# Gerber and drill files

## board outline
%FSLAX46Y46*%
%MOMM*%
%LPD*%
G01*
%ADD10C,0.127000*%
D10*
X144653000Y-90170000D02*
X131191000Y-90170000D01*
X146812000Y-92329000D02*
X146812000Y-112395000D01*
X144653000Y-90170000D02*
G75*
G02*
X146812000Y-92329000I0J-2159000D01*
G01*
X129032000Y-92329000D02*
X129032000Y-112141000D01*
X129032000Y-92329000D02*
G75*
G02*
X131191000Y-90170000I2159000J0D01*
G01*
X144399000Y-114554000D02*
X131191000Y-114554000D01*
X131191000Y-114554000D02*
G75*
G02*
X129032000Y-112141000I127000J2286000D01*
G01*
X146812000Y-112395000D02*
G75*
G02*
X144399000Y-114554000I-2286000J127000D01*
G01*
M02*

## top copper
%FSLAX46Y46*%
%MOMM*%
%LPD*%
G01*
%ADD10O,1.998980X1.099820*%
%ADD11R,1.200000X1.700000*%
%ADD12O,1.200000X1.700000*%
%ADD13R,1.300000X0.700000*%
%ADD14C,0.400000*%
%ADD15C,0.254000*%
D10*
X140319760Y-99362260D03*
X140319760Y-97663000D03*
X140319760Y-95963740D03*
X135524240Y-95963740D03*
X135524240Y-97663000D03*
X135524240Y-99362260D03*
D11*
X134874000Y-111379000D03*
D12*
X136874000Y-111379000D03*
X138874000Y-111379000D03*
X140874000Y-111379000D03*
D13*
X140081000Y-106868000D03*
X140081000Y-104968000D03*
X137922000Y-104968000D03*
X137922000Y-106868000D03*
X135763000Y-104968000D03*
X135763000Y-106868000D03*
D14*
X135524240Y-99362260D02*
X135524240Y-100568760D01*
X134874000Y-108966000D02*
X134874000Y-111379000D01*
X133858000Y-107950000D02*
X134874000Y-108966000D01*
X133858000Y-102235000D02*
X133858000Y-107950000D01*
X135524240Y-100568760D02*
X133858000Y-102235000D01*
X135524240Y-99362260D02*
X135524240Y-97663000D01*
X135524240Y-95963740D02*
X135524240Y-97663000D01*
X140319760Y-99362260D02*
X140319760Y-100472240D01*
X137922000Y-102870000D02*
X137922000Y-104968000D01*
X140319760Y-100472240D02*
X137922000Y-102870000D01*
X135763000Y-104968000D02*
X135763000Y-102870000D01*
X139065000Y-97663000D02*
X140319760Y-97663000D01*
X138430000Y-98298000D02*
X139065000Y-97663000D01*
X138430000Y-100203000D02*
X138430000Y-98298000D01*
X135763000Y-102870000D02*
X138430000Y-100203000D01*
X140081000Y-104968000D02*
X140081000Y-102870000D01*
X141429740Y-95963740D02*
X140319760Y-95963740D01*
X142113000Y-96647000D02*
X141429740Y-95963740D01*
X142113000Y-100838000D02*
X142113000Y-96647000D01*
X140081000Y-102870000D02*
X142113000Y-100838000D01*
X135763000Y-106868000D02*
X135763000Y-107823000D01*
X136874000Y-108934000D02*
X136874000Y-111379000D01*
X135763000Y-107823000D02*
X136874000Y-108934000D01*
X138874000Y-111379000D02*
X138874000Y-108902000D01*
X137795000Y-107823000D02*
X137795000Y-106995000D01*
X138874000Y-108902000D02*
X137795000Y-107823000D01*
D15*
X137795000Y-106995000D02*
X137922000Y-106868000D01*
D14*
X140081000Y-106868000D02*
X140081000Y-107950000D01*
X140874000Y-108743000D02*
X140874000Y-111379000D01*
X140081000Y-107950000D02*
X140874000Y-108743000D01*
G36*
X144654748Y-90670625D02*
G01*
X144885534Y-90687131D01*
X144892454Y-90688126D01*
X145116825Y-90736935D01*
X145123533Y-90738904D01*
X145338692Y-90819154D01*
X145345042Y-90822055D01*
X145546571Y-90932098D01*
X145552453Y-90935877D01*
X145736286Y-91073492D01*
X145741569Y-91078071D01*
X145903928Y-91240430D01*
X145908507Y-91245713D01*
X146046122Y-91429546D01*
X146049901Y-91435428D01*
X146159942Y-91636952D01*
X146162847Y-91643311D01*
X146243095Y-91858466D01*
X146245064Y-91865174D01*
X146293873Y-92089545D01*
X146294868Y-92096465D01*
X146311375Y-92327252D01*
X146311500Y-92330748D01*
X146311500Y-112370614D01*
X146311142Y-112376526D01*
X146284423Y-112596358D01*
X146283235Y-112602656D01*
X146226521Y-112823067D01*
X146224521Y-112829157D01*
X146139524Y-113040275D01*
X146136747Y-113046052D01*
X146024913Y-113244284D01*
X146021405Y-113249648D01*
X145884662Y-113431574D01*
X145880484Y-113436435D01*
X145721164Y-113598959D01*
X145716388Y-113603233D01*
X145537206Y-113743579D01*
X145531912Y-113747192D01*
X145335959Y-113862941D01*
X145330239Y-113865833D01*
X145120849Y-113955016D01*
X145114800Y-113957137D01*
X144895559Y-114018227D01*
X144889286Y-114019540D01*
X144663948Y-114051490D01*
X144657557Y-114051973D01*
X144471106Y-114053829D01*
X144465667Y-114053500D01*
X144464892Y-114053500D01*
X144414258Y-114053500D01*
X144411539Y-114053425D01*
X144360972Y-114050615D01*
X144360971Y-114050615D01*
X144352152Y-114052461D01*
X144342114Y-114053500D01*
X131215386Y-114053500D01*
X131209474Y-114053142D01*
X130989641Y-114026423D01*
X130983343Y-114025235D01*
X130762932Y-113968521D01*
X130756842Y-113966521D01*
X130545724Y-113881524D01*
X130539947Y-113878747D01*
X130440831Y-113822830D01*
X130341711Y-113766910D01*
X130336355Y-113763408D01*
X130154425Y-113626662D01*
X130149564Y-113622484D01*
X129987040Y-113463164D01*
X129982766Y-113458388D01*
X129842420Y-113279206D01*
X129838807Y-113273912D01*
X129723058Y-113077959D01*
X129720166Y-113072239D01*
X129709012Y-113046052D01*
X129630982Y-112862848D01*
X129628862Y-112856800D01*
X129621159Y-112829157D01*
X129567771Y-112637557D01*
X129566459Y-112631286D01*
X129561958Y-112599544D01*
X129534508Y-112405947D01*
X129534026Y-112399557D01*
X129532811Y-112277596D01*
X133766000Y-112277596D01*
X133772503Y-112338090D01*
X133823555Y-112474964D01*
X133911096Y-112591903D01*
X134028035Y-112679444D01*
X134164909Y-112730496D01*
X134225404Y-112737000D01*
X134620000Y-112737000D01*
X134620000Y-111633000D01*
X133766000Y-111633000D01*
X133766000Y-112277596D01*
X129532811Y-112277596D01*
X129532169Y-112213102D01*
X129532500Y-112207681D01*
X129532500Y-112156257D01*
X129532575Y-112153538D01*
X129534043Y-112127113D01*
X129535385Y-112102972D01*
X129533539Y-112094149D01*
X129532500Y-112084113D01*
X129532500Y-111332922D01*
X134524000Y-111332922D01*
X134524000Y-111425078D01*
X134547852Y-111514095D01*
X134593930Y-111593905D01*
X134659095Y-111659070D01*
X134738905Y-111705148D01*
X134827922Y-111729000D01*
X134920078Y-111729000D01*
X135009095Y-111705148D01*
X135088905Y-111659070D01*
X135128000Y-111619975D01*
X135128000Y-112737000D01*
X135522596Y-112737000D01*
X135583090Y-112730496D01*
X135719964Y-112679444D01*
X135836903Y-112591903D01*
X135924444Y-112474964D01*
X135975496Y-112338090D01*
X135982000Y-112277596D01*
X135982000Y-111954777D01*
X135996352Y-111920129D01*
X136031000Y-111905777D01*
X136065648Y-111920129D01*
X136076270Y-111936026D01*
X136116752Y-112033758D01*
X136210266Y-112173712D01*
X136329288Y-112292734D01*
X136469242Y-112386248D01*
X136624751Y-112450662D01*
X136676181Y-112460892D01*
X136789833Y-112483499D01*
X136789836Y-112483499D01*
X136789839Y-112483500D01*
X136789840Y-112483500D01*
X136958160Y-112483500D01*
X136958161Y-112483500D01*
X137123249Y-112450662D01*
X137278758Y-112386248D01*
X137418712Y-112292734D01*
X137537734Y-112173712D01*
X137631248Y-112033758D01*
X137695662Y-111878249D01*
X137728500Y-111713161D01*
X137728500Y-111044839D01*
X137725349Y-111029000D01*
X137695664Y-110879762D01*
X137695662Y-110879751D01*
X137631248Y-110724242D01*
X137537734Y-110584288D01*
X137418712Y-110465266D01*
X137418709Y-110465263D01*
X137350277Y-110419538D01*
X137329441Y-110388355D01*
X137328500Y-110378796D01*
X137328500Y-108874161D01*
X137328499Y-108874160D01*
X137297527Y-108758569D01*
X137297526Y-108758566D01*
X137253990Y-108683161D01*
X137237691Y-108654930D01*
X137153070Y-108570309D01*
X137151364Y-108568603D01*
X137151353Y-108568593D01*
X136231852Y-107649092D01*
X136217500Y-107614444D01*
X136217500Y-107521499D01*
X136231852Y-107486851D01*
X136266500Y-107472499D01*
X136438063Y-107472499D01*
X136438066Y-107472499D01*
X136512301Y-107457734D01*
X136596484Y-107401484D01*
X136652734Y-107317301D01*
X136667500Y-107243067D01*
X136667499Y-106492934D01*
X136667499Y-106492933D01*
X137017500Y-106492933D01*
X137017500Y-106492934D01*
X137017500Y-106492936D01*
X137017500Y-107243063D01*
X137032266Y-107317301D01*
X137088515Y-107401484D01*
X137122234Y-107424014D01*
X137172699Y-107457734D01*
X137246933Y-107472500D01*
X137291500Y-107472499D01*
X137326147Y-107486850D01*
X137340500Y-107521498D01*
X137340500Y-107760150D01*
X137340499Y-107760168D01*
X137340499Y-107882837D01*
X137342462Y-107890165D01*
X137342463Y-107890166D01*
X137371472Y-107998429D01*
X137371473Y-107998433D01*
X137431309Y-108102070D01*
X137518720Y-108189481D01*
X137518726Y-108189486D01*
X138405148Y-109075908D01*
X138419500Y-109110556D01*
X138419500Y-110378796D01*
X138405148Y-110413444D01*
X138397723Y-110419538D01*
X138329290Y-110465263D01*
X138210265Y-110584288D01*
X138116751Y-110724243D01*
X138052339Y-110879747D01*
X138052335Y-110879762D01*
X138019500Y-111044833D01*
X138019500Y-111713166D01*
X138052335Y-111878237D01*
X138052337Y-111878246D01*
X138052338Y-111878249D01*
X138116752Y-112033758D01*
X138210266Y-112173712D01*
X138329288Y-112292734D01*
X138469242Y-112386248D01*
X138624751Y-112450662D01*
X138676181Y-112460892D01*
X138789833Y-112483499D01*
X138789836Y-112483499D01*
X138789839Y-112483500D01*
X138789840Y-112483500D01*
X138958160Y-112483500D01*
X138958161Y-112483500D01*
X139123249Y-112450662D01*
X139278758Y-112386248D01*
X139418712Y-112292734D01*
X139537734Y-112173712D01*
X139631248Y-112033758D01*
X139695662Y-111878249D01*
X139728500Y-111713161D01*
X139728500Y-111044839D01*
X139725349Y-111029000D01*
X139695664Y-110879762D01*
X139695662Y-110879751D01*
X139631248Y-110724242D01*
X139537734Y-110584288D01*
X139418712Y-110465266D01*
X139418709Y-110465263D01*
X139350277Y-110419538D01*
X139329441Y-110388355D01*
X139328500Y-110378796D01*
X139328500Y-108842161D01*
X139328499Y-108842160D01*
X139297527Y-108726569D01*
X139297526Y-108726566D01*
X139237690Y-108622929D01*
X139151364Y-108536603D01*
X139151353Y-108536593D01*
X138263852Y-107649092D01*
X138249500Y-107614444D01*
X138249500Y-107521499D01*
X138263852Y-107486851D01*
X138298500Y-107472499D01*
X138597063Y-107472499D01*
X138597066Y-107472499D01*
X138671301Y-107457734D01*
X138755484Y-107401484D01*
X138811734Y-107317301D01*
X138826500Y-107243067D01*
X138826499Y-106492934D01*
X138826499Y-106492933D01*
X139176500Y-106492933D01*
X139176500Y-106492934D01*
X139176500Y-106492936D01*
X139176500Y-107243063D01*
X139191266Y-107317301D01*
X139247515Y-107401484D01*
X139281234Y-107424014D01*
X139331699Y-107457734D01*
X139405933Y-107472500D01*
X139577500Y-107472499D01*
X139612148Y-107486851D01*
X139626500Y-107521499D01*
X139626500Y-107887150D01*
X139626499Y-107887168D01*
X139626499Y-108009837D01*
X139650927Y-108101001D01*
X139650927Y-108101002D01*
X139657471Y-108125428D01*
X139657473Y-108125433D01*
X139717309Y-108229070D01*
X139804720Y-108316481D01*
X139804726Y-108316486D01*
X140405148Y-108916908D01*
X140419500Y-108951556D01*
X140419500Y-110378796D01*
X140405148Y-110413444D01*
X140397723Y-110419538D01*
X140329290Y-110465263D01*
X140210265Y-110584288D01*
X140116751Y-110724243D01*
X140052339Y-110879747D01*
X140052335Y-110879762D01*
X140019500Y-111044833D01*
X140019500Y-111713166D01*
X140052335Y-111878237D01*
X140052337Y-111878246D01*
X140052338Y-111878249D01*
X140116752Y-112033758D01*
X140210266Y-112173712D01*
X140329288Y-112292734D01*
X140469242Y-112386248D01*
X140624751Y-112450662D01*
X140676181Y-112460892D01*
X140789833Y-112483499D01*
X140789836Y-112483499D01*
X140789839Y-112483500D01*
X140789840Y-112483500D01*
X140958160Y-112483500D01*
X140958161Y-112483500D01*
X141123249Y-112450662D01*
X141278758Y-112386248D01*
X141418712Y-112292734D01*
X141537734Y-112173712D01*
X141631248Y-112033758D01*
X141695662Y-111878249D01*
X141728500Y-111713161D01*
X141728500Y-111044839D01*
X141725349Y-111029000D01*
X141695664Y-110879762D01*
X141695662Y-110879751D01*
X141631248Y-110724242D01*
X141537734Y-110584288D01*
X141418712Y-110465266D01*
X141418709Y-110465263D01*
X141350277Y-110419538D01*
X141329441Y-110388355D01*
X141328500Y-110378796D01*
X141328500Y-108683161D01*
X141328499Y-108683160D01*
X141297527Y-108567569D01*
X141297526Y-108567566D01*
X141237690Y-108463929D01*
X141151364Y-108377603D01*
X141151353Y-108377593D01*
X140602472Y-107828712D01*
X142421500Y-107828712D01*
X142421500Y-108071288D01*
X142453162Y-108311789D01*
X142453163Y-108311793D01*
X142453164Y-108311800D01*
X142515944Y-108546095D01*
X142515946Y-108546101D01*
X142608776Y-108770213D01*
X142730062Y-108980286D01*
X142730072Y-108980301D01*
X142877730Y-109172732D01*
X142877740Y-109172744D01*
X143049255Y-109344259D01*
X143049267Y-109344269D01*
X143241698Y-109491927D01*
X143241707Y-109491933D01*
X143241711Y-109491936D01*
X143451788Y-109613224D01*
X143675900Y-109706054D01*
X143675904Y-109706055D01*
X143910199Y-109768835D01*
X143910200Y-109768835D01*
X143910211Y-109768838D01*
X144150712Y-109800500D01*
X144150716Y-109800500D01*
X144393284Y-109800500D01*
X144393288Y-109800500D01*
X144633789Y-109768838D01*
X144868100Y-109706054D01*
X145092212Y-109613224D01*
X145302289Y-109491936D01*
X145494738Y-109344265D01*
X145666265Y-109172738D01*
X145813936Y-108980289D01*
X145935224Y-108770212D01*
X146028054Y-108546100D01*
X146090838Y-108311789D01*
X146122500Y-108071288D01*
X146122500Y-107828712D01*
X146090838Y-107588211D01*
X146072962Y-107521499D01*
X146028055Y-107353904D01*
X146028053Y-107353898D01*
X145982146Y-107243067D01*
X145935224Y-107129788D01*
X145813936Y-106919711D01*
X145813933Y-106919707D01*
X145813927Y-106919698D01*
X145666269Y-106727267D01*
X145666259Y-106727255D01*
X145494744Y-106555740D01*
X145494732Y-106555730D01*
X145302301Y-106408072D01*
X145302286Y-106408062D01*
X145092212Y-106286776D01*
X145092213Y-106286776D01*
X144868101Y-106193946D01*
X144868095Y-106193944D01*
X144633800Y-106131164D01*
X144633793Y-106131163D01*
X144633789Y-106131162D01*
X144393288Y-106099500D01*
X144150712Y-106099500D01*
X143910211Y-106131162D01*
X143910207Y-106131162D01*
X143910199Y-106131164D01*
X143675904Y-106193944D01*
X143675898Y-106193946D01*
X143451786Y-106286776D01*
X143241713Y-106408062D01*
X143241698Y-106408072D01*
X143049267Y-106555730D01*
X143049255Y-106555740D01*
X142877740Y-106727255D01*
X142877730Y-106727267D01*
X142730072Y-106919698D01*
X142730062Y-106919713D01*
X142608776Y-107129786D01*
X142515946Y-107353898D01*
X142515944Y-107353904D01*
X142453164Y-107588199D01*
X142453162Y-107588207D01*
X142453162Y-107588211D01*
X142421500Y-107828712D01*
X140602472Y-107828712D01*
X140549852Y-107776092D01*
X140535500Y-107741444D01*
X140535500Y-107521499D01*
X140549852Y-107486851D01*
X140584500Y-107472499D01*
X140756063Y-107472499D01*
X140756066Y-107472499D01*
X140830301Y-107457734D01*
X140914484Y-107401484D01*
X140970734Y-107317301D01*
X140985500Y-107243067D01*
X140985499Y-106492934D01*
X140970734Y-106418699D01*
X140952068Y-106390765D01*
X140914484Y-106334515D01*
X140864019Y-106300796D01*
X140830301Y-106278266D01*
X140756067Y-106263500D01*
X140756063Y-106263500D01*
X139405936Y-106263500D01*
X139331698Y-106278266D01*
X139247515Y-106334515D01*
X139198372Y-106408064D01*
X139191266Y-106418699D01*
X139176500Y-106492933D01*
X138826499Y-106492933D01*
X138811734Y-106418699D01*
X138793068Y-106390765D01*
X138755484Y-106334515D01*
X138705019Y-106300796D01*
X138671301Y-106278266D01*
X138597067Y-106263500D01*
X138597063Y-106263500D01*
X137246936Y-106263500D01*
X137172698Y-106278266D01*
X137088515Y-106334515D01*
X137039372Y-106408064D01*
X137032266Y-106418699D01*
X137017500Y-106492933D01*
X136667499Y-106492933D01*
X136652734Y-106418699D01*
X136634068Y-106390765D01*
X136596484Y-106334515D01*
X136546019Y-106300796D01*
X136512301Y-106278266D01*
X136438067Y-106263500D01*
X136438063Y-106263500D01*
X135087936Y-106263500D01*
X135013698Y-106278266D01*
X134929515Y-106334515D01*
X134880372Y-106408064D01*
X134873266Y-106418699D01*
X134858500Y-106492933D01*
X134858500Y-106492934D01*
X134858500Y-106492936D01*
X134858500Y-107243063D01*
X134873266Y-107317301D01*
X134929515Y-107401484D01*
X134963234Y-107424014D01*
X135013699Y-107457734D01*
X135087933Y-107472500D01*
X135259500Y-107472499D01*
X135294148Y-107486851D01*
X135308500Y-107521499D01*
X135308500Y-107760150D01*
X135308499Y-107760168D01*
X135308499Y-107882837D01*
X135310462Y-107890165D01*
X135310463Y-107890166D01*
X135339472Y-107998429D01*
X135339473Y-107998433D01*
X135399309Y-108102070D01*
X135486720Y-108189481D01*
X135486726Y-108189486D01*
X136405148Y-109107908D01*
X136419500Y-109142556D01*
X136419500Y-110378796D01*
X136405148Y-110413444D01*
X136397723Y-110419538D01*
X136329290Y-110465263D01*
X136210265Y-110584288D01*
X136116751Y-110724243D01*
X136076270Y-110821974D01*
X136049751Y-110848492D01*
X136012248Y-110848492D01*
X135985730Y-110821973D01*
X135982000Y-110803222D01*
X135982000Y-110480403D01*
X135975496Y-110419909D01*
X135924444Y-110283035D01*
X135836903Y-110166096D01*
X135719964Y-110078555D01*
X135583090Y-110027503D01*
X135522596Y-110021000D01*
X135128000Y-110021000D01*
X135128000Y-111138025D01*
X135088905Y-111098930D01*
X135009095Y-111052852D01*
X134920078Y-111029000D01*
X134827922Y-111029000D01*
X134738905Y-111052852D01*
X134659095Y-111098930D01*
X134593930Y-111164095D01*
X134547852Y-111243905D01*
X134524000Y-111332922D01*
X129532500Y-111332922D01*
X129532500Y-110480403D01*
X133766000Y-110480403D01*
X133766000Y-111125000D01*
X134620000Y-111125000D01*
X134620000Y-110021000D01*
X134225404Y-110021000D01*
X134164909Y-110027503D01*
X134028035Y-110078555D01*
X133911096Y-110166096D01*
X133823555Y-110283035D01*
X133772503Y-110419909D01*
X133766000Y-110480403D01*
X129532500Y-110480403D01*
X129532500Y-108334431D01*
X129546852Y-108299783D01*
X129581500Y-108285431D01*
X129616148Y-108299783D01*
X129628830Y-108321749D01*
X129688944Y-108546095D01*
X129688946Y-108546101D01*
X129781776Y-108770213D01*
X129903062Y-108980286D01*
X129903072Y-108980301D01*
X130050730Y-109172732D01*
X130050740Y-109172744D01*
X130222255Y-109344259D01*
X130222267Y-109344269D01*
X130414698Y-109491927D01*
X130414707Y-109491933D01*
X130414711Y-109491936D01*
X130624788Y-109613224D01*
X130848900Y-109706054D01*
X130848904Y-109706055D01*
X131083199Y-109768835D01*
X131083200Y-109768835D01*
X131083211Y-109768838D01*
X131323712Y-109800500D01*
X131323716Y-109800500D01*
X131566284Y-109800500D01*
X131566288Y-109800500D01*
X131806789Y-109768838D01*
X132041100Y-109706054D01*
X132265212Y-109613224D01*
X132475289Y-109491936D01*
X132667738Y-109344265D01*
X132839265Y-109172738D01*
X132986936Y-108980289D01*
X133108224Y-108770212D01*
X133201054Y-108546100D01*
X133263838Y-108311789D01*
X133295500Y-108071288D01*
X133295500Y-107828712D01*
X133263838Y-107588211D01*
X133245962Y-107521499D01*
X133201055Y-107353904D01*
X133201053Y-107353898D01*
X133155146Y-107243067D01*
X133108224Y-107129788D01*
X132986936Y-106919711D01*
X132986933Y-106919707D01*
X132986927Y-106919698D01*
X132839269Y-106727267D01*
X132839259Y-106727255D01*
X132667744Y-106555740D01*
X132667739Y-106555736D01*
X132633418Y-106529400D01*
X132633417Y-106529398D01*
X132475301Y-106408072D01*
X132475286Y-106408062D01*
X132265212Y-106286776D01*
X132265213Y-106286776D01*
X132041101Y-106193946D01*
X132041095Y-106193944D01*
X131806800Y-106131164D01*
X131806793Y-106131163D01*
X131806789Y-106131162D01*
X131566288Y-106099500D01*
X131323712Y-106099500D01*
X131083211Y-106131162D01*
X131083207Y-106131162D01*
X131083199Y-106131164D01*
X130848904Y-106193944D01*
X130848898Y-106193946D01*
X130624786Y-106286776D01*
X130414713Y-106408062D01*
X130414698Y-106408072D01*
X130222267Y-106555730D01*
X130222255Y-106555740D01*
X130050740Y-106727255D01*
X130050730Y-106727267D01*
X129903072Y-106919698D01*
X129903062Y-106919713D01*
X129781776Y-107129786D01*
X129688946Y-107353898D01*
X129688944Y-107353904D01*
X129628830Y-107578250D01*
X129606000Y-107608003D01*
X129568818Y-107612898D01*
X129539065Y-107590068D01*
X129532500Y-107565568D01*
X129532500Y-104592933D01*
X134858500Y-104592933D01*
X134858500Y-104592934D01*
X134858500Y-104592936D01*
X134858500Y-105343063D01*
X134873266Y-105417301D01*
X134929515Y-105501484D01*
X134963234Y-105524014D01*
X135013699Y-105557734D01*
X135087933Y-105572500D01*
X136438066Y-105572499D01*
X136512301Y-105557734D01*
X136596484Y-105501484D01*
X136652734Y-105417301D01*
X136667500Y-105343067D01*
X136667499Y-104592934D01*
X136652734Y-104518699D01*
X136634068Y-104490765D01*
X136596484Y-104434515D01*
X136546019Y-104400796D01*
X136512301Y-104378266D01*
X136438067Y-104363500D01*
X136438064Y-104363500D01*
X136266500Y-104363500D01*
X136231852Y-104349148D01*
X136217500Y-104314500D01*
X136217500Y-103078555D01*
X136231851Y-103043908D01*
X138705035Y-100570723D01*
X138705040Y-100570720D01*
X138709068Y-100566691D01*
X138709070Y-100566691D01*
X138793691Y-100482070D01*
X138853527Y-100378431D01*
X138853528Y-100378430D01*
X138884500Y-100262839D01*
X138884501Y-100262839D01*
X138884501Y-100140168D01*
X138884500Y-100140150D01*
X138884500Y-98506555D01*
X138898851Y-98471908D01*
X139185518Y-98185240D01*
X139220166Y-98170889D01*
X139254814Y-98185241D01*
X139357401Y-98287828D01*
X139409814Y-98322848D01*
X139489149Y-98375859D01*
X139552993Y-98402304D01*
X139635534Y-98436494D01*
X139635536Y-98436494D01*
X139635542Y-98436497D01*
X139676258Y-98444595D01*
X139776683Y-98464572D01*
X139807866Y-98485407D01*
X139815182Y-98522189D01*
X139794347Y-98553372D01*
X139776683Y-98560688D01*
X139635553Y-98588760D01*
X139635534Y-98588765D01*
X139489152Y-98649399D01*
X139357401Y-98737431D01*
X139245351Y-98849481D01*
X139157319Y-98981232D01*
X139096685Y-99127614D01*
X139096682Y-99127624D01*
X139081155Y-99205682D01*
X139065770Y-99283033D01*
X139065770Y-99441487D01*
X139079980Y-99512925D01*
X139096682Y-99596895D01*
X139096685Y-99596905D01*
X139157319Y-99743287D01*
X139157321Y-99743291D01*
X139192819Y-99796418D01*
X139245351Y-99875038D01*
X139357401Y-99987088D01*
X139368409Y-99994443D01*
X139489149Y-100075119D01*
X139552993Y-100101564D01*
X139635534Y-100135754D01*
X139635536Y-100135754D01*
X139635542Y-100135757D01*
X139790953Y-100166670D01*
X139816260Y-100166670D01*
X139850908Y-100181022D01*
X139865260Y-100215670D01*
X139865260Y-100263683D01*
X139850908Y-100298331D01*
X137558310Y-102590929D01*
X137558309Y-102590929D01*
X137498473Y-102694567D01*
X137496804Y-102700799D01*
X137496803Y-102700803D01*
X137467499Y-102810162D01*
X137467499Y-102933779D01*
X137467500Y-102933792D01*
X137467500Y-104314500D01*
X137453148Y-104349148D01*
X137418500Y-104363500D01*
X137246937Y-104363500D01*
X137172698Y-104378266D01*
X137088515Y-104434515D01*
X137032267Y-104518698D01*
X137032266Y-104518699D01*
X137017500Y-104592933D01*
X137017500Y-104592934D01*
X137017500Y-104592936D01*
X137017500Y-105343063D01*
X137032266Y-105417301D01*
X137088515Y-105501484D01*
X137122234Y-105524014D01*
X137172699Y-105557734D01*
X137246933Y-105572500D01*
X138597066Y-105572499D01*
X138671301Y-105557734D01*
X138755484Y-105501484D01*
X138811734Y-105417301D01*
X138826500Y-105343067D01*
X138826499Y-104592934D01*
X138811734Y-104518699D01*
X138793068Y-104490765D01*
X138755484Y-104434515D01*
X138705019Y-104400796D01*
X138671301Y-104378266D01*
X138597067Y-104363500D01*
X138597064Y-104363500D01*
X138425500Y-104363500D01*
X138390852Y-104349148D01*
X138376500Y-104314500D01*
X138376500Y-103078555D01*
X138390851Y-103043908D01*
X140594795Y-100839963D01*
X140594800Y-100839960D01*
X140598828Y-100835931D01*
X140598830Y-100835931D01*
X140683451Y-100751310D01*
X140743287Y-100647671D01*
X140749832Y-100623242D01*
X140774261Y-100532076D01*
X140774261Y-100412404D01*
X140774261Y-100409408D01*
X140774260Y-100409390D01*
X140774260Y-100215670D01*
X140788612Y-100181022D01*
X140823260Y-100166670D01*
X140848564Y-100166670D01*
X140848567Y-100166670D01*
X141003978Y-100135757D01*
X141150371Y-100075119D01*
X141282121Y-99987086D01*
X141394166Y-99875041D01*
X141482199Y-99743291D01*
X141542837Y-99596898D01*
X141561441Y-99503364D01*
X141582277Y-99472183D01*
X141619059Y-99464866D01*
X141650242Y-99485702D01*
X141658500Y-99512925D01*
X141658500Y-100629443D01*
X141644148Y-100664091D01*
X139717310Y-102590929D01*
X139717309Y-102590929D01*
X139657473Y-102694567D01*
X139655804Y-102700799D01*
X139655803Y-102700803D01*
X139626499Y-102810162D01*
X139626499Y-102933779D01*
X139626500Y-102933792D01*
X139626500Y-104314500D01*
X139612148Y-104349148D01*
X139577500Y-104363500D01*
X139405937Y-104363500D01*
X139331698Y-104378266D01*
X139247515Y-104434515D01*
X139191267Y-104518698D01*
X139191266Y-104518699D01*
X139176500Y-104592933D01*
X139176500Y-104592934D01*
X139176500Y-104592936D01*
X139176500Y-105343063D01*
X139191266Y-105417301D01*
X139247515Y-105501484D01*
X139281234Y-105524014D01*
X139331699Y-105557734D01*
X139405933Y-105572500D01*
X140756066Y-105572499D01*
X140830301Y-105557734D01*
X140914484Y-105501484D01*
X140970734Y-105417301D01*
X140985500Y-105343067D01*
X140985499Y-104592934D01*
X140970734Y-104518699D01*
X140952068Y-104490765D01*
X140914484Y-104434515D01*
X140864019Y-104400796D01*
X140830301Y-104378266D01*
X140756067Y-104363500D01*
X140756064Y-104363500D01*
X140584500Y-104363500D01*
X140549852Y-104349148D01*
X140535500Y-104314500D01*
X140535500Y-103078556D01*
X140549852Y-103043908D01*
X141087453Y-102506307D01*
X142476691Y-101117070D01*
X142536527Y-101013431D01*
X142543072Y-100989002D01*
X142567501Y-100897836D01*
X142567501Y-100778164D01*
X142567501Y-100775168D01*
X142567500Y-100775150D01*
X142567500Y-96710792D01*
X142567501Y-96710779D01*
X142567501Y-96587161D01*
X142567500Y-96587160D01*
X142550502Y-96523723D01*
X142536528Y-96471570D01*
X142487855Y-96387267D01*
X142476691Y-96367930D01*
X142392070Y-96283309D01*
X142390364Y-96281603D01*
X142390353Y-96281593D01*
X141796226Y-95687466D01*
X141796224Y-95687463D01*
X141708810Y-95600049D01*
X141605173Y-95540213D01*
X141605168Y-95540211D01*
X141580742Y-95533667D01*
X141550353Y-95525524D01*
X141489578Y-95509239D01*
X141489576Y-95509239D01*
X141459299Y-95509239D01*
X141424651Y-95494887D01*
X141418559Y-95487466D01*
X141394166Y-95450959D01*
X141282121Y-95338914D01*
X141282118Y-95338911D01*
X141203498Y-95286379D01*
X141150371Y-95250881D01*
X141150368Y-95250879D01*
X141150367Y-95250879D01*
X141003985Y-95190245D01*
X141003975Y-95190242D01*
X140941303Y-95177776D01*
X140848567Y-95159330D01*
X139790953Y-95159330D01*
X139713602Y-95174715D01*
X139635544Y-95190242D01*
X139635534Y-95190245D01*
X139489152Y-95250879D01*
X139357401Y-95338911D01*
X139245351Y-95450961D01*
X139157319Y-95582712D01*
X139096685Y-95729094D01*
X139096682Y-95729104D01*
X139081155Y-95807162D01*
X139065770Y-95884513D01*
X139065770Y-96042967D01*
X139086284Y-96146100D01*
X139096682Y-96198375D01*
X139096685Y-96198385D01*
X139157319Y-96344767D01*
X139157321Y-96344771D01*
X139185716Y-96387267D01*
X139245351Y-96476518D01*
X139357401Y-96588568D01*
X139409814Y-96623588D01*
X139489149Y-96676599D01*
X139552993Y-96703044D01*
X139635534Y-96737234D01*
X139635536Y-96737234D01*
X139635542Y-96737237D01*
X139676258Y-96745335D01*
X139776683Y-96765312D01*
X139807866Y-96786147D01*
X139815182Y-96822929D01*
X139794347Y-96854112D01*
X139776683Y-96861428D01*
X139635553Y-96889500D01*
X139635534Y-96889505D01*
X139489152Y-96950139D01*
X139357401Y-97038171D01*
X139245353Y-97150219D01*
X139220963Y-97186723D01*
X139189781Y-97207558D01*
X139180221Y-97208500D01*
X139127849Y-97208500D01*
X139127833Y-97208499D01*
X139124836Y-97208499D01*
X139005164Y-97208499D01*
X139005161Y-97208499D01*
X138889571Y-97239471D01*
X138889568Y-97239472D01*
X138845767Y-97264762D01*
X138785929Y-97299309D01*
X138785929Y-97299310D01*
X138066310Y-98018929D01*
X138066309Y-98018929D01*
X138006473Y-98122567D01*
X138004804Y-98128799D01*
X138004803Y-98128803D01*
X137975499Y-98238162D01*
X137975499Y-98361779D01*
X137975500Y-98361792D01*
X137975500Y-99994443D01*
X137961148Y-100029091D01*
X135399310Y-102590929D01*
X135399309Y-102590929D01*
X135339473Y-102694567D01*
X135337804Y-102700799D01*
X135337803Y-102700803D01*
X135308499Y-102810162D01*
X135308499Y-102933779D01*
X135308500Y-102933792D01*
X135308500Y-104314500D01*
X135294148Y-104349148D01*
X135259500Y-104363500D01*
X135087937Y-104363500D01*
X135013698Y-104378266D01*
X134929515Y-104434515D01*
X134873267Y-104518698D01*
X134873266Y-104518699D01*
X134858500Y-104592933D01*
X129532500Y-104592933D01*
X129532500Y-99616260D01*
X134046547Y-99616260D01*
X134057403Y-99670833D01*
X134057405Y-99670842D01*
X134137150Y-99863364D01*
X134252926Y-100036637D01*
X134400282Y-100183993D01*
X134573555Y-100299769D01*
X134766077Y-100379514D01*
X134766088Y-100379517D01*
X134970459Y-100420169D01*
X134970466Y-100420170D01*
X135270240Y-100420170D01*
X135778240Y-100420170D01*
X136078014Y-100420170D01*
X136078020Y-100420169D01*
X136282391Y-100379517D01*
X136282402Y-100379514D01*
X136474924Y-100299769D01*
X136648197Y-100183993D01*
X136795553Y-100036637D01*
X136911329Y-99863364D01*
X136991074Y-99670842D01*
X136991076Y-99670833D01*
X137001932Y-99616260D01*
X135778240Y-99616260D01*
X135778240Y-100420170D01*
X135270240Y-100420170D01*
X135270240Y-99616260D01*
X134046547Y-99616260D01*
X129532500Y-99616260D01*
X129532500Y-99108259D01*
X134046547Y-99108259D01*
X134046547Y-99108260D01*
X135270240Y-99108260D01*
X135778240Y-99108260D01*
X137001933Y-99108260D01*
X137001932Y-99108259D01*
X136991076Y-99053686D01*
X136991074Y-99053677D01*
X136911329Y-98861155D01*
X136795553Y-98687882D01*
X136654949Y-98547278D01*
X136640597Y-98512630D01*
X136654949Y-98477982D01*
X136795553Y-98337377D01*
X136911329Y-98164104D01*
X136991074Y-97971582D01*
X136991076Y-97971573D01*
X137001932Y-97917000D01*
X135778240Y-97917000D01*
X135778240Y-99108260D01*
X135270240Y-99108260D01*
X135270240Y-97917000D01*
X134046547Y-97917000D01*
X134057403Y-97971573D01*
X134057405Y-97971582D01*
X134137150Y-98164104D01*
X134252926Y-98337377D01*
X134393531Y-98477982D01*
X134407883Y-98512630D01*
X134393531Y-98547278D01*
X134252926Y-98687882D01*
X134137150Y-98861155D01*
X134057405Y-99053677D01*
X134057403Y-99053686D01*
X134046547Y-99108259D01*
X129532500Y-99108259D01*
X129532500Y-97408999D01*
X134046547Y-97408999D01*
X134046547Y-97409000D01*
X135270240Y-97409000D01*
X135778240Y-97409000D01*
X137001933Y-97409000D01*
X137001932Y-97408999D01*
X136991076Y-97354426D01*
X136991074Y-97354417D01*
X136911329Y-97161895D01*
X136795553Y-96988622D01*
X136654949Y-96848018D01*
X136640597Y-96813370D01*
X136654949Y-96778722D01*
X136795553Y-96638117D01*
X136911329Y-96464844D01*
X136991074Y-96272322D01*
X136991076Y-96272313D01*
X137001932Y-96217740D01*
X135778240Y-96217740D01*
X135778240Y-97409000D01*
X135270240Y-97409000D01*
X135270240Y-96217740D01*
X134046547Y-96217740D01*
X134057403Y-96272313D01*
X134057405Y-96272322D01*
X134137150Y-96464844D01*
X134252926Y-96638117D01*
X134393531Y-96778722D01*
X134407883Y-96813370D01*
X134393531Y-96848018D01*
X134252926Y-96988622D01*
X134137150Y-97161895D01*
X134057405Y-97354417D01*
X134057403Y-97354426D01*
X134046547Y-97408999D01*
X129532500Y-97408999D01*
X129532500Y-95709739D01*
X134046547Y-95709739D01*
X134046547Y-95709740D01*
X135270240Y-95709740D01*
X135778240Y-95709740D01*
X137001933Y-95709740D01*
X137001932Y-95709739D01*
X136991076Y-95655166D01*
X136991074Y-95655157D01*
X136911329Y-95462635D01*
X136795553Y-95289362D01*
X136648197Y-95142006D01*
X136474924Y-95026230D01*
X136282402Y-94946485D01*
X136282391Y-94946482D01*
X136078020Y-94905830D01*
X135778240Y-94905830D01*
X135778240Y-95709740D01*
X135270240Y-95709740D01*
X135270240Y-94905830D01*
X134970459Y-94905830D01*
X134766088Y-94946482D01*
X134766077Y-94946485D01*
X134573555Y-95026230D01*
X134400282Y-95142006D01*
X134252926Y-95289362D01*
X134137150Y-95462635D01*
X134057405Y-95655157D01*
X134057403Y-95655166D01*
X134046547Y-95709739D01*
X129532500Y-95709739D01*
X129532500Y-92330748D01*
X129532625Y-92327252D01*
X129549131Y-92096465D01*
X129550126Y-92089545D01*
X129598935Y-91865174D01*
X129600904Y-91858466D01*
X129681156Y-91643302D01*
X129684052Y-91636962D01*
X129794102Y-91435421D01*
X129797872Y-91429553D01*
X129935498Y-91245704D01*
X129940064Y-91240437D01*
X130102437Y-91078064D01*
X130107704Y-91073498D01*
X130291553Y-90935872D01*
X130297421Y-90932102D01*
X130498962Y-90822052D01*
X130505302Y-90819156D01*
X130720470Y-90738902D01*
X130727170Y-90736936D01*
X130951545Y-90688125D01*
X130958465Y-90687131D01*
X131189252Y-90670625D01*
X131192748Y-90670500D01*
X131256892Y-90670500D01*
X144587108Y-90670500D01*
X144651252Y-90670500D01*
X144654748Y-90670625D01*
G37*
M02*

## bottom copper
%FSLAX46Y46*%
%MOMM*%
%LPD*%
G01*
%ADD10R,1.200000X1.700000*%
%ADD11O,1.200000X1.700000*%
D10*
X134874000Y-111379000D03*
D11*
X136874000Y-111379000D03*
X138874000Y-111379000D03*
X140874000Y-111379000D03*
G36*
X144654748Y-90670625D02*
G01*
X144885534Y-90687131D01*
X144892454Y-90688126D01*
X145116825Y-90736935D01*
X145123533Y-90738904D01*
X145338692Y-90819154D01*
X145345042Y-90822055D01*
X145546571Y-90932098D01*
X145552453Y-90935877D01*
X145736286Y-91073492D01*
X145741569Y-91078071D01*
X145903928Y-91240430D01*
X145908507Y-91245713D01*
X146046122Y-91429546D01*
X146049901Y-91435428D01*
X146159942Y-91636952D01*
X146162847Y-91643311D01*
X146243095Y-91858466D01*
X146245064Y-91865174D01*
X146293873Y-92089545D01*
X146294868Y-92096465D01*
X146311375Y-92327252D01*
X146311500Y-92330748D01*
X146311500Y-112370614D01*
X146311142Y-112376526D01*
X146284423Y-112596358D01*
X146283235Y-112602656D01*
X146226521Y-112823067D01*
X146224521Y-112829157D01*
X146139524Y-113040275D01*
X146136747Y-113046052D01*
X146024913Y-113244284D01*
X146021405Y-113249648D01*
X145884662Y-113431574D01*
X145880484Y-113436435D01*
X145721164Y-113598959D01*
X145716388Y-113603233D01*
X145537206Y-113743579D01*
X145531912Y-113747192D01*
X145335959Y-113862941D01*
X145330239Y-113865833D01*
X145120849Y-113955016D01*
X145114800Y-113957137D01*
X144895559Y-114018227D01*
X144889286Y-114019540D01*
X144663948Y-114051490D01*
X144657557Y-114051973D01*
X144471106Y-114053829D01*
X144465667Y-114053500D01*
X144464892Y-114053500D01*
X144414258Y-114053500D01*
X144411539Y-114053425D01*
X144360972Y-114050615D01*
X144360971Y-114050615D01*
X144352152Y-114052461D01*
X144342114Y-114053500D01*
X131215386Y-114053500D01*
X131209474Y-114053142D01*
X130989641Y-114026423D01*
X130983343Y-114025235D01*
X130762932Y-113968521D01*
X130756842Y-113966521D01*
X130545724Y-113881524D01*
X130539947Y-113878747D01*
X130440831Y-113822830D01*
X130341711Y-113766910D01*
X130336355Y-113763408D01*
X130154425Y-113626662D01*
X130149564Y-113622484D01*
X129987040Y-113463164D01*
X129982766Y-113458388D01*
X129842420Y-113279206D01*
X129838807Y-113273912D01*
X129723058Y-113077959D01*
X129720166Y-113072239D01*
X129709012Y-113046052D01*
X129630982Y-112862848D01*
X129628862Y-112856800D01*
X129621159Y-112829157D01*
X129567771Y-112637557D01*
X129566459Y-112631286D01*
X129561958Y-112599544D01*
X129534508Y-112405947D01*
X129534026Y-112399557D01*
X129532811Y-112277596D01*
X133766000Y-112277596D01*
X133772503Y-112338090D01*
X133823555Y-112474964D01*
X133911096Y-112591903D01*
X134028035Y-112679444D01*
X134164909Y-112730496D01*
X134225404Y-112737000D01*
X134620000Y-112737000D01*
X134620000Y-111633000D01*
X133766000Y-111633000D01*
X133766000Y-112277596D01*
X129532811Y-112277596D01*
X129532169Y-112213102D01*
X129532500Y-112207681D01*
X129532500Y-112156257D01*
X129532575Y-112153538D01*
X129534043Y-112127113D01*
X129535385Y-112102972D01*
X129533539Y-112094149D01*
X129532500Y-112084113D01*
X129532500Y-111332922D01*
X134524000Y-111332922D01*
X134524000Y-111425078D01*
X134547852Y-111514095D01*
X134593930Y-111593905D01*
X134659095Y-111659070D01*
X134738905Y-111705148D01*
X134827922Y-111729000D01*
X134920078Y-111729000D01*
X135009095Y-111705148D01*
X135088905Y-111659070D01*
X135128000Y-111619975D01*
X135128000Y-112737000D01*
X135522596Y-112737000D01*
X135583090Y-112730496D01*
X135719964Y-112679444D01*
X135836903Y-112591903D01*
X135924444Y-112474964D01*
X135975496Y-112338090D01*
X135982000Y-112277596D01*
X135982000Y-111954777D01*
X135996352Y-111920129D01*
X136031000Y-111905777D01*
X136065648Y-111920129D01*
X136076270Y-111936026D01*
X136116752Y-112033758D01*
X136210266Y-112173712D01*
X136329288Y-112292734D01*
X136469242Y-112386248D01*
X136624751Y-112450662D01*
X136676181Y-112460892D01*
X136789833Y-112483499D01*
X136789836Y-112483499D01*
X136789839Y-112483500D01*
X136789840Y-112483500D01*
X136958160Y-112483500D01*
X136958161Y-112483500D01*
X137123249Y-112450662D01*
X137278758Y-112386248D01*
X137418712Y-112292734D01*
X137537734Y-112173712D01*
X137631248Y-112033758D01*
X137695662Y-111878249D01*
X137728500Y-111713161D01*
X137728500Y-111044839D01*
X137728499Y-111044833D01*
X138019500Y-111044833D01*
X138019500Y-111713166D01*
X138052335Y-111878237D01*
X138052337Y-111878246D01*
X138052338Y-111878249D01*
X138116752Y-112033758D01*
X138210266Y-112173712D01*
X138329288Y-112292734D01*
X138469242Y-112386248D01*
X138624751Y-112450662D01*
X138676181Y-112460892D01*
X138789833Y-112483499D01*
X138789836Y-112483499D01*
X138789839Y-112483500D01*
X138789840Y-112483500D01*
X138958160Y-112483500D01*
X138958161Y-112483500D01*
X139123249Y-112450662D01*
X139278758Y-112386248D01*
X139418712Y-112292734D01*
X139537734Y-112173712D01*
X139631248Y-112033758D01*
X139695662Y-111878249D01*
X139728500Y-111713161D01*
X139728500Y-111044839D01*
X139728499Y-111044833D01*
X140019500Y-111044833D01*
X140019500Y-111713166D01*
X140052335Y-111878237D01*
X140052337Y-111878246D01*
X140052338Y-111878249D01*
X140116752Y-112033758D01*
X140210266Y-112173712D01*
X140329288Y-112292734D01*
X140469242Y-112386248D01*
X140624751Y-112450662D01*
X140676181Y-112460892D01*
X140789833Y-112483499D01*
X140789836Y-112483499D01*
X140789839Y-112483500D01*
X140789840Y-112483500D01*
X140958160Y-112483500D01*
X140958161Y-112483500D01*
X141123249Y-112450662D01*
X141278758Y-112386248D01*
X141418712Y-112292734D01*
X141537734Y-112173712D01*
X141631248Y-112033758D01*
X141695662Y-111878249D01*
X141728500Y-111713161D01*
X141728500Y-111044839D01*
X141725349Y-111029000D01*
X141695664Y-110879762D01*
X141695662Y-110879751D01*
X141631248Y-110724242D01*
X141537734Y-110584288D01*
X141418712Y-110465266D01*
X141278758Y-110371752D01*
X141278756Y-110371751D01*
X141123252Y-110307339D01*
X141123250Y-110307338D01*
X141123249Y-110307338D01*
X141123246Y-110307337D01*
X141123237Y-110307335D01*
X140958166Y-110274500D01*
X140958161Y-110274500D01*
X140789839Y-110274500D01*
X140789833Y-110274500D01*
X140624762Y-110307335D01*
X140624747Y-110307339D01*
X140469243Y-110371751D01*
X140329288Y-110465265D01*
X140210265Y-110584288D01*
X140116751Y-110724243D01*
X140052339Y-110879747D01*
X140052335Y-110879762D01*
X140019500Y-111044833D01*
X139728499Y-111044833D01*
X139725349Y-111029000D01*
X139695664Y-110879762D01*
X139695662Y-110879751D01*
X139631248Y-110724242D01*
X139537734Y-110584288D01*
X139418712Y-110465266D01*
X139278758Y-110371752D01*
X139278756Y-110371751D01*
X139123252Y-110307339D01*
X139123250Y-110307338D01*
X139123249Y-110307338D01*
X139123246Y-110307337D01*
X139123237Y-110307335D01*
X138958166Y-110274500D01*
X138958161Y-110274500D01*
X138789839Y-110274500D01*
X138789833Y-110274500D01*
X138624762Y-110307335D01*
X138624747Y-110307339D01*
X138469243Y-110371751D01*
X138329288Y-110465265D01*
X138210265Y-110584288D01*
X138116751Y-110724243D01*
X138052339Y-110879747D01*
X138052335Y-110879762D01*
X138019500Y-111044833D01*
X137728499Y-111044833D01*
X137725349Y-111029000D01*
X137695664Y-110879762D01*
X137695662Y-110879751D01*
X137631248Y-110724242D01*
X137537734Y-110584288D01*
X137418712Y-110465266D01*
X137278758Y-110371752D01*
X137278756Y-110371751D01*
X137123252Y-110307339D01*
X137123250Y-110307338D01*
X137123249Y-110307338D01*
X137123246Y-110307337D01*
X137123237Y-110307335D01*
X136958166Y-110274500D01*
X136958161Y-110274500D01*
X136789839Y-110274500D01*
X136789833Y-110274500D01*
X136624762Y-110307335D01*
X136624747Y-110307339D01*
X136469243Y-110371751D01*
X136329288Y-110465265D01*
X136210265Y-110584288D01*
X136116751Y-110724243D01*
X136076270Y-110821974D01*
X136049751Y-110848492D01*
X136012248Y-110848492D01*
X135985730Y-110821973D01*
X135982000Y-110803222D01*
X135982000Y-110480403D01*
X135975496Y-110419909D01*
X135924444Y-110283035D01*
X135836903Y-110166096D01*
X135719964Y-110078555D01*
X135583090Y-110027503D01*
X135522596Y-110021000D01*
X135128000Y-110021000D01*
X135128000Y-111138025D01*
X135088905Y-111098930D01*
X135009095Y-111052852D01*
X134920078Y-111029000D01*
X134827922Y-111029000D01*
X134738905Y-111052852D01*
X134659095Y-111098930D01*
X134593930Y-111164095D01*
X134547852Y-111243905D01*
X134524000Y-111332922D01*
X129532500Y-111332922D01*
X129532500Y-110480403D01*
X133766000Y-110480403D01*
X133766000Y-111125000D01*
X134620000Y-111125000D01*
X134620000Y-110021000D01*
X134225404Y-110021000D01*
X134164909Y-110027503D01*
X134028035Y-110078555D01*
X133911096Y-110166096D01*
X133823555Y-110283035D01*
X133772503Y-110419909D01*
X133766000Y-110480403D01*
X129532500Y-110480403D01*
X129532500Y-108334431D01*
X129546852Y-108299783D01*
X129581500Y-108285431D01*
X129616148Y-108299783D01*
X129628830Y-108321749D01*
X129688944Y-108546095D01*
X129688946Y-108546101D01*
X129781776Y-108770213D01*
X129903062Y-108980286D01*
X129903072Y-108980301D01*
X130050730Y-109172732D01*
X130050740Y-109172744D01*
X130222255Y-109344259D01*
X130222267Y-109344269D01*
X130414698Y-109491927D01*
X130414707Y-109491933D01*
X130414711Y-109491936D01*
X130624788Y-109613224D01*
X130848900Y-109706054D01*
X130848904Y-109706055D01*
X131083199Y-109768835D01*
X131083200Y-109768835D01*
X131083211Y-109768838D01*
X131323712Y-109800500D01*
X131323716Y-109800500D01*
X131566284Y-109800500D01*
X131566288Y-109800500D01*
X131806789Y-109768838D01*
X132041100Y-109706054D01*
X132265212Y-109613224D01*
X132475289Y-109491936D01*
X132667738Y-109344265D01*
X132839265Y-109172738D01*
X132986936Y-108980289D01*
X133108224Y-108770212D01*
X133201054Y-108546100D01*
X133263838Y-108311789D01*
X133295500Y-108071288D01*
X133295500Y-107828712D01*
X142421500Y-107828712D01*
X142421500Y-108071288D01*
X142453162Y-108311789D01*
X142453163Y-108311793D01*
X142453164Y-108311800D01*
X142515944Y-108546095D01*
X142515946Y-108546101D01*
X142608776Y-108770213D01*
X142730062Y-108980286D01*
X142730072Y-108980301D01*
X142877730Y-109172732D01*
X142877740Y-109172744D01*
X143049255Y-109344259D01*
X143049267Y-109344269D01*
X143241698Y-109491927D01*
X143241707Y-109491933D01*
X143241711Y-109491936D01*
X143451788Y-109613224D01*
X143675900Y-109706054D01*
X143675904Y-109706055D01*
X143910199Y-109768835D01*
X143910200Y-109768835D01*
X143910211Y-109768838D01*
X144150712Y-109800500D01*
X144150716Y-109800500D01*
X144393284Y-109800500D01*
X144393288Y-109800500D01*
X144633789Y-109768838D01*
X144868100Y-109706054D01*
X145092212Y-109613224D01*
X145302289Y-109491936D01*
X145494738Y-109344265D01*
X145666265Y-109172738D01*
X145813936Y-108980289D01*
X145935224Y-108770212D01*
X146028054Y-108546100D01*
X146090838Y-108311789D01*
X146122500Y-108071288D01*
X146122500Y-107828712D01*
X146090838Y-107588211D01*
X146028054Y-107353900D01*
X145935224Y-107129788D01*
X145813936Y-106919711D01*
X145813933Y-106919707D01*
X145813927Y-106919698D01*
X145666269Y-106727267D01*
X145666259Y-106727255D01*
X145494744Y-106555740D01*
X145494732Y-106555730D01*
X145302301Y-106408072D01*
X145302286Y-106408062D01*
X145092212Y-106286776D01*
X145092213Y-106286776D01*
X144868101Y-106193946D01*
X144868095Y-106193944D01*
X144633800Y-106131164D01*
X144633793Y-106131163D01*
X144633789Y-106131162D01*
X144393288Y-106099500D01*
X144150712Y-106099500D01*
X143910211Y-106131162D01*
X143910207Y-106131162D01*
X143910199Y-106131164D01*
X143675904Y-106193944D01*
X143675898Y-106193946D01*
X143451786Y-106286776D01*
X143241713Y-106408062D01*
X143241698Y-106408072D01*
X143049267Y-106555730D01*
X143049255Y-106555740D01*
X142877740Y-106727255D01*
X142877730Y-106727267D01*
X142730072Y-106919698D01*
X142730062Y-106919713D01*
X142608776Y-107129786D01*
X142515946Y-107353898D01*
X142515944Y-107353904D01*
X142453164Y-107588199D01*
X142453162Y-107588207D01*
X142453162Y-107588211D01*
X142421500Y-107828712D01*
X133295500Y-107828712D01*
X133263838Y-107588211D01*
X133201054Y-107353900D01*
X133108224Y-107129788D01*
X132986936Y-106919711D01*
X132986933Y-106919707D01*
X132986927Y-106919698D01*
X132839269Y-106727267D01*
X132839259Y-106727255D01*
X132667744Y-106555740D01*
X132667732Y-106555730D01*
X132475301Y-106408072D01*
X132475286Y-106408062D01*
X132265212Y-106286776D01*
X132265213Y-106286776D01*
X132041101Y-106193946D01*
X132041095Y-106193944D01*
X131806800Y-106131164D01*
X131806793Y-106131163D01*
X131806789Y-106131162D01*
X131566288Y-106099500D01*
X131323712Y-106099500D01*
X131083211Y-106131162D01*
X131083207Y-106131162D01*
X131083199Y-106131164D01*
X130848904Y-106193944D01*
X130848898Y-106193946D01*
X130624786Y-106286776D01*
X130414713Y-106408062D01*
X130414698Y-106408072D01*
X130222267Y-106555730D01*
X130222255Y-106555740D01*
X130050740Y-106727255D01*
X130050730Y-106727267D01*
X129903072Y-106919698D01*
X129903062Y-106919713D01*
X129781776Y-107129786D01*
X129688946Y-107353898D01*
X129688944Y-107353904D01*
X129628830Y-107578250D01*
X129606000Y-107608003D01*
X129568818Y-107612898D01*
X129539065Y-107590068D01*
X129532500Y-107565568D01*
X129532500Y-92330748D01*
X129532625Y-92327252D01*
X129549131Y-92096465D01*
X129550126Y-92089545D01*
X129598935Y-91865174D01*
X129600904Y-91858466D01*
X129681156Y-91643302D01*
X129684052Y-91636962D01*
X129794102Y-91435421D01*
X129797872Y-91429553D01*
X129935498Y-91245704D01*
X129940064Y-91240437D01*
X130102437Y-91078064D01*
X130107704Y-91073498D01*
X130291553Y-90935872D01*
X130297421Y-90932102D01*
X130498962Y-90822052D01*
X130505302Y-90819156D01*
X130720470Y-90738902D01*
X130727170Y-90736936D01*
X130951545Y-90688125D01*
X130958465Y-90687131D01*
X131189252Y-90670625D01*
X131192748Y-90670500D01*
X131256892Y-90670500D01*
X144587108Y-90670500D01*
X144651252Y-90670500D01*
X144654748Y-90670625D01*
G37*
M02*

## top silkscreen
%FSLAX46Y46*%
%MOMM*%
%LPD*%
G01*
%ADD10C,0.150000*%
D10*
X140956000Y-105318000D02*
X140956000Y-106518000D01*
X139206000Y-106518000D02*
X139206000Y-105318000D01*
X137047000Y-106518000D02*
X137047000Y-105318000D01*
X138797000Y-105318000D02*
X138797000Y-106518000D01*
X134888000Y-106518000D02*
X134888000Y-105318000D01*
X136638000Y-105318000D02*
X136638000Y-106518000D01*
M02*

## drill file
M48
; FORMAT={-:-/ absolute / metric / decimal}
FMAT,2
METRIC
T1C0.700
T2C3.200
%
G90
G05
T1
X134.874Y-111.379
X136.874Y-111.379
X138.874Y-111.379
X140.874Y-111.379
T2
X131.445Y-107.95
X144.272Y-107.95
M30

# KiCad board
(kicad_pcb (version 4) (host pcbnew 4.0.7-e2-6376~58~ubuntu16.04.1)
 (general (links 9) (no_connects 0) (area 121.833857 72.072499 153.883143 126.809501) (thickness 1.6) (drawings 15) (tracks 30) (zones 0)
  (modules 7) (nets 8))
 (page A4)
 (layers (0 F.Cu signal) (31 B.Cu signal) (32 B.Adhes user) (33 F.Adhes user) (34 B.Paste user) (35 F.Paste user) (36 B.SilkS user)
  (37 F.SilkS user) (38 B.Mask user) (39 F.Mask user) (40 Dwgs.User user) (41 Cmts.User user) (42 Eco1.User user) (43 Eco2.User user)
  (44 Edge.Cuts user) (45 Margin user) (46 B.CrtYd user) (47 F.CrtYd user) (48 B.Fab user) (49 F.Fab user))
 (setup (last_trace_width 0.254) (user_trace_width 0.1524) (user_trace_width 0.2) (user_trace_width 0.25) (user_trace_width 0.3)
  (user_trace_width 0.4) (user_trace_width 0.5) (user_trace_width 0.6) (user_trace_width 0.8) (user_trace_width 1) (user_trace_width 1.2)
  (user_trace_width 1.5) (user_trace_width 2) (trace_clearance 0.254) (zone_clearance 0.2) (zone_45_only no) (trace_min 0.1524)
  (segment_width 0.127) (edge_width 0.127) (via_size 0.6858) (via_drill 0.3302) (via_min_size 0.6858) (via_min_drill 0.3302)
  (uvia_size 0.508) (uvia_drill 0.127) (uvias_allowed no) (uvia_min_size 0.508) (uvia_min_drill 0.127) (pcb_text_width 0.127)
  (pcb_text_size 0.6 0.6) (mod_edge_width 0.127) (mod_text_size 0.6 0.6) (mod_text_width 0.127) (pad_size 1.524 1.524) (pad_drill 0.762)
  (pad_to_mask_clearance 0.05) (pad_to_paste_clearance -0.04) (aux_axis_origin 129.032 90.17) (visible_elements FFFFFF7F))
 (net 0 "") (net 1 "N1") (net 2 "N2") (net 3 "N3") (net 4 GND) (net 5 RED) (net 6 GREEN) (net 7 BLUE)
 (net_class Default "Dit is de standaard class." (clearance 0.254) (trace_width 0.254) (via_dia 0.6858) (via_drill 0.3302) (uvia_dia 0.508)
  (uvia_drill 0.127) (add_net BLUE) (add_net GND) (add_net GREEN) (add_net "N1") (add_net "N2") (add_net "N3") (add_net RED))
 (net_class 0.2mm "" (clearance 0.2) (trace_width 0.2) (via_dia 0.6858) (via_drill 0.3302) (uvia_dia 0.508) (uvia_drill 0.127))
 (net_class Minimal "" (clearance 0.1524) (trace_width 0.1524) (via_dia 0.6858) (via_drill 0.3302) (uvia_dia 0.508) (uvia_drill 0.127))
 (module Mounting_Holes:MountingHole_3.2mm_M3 (layer F.Cu) (at 144.272 107.95)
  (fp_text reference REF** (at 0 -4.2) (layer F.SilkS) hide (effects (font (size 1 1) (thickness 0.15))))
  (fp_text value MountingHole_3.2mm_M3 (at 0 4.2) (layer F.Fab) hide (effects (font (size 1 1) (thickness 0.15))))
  (pad 1 np_thru_hole circle (at 0 0) (size 3.2 3.2) (drill 3.2) (layers *.Cu *.Mask)))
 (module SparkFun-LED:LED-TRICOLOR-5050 (layer F.Cu) (at 137.922 97.663 180)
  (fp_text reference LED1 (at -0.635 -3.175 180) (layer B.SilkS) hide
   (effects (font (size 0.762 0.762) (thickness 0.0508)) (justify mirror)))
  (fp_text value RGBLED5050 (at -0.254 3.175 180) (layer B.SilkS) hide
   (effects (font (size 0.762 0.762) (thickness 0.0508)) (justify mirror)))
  (pad 1 smd oval (at -2.39776 -1.69926 180) (size 1.99898 1.09982) (layers F.Cu F.Paste F.Mask) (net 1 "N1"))
  (pad 2 smd oval (at -2.39776 0 180) (size 1.99898 1.09982) (layers F.Cu F.Paste F.Mask) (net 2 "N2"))
  (pad 3 smd oval (at -2.39776 1.69926 180) (size 1.99898 1.09982) (layers F.Cu F.Paste F.Mask) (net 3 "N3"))
  (pad 4 smd oval (at 2.39776 1.69926 180) (size 1.99898 1.09982) (layers F.Cu F.Paste F.Mask) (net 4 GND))
  (pad 5 smd oval (at 2.39776 0 180) (size 1.99898 1.09982) (layers F.Cu F.Paste F.Mask) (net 4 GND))
  (pad 6 smd oval (at 2.39776 -1.69926 180) (size 1.99898 1.09982) (layers F.Cu F.Paste F.Mask) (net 4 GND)))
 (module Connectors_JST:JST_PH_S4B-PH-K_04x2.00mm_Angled (layer F.Cu) (at 134.874 111.379)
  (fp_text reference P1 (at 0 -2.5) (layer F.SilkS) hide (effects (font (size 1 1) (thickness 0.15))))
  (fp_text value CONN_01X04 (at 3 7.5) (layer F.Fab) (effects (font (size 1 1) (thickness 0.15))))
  (pad 1 thru_hole rect (at 0 0) (size 1.2 1.7) (drill 0.7) (layers *.Cu *.Mask) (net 4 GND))
  (pad 2 thru_hole oval (at 2 0) (size 1.2 1.7) (drill 0.7) (layers *.Cu *.Mask) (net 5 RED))
  (pad 3 thru_hole oval (at 4 0) (size 1.2 1.7) (drill 0.7) (layers *.Cu *.Mask) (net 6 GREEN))
  (pad 4 thru_hole oval (at 6 0) (size 1.2 1.7) (drill 0.7) (layers *.Cu *.Mask) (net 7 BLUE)))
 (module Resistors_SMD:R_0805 (layer F.Cu) (at 140.081 105.918 90)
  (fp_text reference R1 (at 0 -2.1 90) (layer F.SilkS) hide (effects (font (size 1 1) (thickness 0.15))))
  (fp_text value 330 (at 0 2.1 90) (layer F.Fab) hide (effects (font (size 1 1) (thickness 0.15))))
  (fp_line (start 0.6 0.875) (end -0.6 0.875) (layer F.SilkS) (width 0.15))
  (fp_line (start -0.6 -0.875) (end 0.6 -0.875) (layer F.SilkS) (width 0.15))
  (pad 1 smd rect (at -0.95 0 90) (size 0.7 1.3) (layers F.Cu F.Paste F.Mask) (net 7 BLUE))
  (pad 2 smd rect (at 0.95 0 90) (size 0.7 1.3) (layers F.Cu F.Paste F.Mask) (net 3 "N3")))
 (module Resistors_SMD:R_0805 (layer F.Cu) (at 137.922 105.918 270)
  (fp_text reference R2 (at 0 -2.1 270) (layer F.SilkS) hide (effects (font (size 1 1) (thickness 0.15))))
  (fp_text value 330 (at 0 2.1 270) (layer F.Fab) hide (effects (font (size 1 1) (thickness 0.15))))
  (fp_line (start 0.6 0.875) (end -0.6 0.875) (layer F.SilkS) (width 0.15))
  (fp_line (start -0.6 -0.875) (end 0.6 -0.875) (layer F.SilkS) (width 0.15))
  (pad 1 smd rect (at -0.95 0 270) (size 0.7 1.3) (layers F.Cu F.Paste F.Mask) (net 1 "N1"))
  (pad 2 smd rect (at 0.95 0 270) (size 0.7 1.3) (layers F.Cu F.Paste F.Mask) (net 6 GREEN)))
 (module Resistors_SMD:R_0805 (layer F.Cu) (at 135.763 105.918 270)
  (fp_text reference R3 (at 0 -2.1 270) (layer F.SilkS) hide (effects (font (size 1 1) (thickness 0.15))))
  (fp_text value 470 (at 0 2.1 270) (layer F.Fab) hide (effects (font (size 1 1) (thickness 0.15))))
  (fp_line (start 0.6 0.875) (end -0.6 0.875) (layer F.SilkS) (width 0.15))
  (fp_line (start -0.6 -0.875) (end 0.6 -0.875) (layer F.SilkS) (width 0.15))
  (pad 1 smd rect (at -0.95 0 270) (size 0.7 1.3) (layers F.Cu F.Paste F.Mask) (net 2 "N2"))
  (pad 2 smd rect (at 0.95 0 270) (size 0.7 1.3) (layers F.Cu F.Paste F.Mask) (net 5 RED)))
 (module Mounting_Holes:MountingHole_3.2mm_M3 (layer F.Cu) (at 131.445 107.95)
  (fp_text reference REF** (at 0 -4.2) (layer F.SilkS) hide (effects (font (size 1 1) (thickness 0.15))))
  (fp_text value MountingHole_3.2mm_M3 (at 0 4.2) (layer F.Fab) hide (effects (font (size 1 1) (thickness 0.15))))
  (pad 1 np_thru_hole circle (at 0 0) (size 3.2 3.2) (drill 3.2) (layers *.Cu *.Mask)))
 (gr_line (start 144.653 90.17) (end 131.191 90.17) (angle 90) (layer Edge.Cuts) (width 0.127))
 (gr_line (start 146.812 92.329) (end 146.812 112.395) (angle 90) (layer Edge.Cuts) (width 0.127))
 (gr_arc (start 144.653 92.329) (end 144.653 90.17) (angle 90) (layer Edge.Cuts) (width 0.127))
 (gr_line (start 129.032 92.329) (end 129.032 112.141) (angle 90) (layer Edge.Cuts) (width 0.127))
 (gr_arc (start 131.191 92.329) (end 129.032 92.329) (angle 90) (layer Edge.Cuts) (width 0.127))
 (gr_line (start 144.399 114.554) (end 131.191 114.554) (angle 90) (layer Edge.Cuts) (width 0.127))
 (gr_arc (start 131.318 112.268) (end 131.191 114.554) (angle 90) (layer Edge.Cuts) (width 0.127))
 (gr_arc (start 144.526 112.268) (end 146.812 112.395) (angle 90) (layer Edge.Cuts) (width 0.127))
 (segment (start 135.52424 99.36226) (end 135.52424 100.56876) (width 0.4) (layer F.Cu) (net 4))
 (segment (start 134.874 108.966) (end 134.874 111.379) (width 0.4) (layer F.Cu) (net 4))
 (segment (start 133.858 107.95) (end 134.874 108.966) (width 0.4) (layer F.Cu) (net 4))
 (segment (start 133.858 102.235) (end 133.858 107.95) (width 0.4) (layer F.Cu) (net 4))
 (segment (start 135.52424 100.56876) (end 133.858 102.235) (width 0.4) (layer F.Cu) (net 4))
 (segment (start 135.52424 99.36226) (end 135.52424 97.663) (width 0.4) (layer F.Cu) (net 4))
 (segment (start 135.52424 95.96374) (end 135.52424 97.663) (width 0.4) (layer F.Cu) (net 4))
 (segment (start 140.31976 99.36226) (end 140.31976 100.47224) (width 0.4) (layer F.Cu) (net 1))
 (segment (start 137.922 102.87) (end 137.922 104.968) (width 0.4) (layer F.Cu) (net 1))
 (segment (start 140.31976 100.47224) (end 137.922 102.87) (width 0.4) (layer F.Cu) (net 1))
 (segment (start 135.763 104.968) (end 135.763 102.87) (width 0.4) (layer F.Cu) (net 2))
 (segment (start 139.065 97.663) (end 140.31976 97.663) (width 0.4) (layer F.Cu) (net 2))
 (segment (start 138.43 98.298) (end 139.065 97.663) (width 0.4) (layer F.Cu) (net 2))
 (segment (start 138.43 100.203) (end 138.43 98.298) (width 0.4) (layer F.Cu) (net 2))
 (segment (start 135.763 102.87) (end 138.43 100.203) (width 0.4) (layer F.Cu) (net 2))
 (segment (start 140.081 104.968) (end 140.081 102.87) (width 0.4) (layer F.Cu) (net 3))
 (segment (start 141.42974 95.96374) (end 140.31976 95.96374) (width 0.4) (layer F.Cu) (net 3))
 (segment (start 142.113 96.647) (end 141.42974 95.96374) (width 0.4) (layer F.Cu) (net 3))
 (segment (start 142.113 100.838) (end 142.113 96.647) (width 0.4) (layer F.Cu) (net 3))
 (segment (start 140.081 102.87) (end 142.113 100.838) (width 0.4) (layer F.Cu) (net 3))
 (segment (start 135.763 106.868) (end 135.763 107.823) (width 0.4) (layer F.Cu) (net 5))
 (segment (start 136.874 108.934) (end 136.874 111.379) (width 0.4) (layer F.Cu) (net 5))
 (segment (start 135.763 107.823) (end 136.874 108.934) (width 0.4) (layer F.Cu) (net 5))
 (segment (start 138.874 111.379) (end 138.874 108.902) (width 0.4) (layer F.Cu) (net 6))
 (segment (start 137.795 107.823) (end 137.795 106.995) (width 0.4) (layer F.Cu) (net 6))
 (segment (start 138.874 108.902) (end 137.795 107.823) (width 0.4) (layer F.Cu) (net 6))
 (segment (start 137.795 106.995) (end 137.922 106.868) (width 0.254) (layer F.Cu) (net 6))
 (segment (start 140.081 106.868) (end 140.081 107.95) (width 0.4) (layer F.Cu) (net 7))
 (segment (start 140.874 108.743) (end 140.874 111.379) (width 0.4) (layer F.Cu) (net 7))
 (segment (start 140.081 107.95) (end 140.874 108.743) (width 0.4) (layer F.Cu) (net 7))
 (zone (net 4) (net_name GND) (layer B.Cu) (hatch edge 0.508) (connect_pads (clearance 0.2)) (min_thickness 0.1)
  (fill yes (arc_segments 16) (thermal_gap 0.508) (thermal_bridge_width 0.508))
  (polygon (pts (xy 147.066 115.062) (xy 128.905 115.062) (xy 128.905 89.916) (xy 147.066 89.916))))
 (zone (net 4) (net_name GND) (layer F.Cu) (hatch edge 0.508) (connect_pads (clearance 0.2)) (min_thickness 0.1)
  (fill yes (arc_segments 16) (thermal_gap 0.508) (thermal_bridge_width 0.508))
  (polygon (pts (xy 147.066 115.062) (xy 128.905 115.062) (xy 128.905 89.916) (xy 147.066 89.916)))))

